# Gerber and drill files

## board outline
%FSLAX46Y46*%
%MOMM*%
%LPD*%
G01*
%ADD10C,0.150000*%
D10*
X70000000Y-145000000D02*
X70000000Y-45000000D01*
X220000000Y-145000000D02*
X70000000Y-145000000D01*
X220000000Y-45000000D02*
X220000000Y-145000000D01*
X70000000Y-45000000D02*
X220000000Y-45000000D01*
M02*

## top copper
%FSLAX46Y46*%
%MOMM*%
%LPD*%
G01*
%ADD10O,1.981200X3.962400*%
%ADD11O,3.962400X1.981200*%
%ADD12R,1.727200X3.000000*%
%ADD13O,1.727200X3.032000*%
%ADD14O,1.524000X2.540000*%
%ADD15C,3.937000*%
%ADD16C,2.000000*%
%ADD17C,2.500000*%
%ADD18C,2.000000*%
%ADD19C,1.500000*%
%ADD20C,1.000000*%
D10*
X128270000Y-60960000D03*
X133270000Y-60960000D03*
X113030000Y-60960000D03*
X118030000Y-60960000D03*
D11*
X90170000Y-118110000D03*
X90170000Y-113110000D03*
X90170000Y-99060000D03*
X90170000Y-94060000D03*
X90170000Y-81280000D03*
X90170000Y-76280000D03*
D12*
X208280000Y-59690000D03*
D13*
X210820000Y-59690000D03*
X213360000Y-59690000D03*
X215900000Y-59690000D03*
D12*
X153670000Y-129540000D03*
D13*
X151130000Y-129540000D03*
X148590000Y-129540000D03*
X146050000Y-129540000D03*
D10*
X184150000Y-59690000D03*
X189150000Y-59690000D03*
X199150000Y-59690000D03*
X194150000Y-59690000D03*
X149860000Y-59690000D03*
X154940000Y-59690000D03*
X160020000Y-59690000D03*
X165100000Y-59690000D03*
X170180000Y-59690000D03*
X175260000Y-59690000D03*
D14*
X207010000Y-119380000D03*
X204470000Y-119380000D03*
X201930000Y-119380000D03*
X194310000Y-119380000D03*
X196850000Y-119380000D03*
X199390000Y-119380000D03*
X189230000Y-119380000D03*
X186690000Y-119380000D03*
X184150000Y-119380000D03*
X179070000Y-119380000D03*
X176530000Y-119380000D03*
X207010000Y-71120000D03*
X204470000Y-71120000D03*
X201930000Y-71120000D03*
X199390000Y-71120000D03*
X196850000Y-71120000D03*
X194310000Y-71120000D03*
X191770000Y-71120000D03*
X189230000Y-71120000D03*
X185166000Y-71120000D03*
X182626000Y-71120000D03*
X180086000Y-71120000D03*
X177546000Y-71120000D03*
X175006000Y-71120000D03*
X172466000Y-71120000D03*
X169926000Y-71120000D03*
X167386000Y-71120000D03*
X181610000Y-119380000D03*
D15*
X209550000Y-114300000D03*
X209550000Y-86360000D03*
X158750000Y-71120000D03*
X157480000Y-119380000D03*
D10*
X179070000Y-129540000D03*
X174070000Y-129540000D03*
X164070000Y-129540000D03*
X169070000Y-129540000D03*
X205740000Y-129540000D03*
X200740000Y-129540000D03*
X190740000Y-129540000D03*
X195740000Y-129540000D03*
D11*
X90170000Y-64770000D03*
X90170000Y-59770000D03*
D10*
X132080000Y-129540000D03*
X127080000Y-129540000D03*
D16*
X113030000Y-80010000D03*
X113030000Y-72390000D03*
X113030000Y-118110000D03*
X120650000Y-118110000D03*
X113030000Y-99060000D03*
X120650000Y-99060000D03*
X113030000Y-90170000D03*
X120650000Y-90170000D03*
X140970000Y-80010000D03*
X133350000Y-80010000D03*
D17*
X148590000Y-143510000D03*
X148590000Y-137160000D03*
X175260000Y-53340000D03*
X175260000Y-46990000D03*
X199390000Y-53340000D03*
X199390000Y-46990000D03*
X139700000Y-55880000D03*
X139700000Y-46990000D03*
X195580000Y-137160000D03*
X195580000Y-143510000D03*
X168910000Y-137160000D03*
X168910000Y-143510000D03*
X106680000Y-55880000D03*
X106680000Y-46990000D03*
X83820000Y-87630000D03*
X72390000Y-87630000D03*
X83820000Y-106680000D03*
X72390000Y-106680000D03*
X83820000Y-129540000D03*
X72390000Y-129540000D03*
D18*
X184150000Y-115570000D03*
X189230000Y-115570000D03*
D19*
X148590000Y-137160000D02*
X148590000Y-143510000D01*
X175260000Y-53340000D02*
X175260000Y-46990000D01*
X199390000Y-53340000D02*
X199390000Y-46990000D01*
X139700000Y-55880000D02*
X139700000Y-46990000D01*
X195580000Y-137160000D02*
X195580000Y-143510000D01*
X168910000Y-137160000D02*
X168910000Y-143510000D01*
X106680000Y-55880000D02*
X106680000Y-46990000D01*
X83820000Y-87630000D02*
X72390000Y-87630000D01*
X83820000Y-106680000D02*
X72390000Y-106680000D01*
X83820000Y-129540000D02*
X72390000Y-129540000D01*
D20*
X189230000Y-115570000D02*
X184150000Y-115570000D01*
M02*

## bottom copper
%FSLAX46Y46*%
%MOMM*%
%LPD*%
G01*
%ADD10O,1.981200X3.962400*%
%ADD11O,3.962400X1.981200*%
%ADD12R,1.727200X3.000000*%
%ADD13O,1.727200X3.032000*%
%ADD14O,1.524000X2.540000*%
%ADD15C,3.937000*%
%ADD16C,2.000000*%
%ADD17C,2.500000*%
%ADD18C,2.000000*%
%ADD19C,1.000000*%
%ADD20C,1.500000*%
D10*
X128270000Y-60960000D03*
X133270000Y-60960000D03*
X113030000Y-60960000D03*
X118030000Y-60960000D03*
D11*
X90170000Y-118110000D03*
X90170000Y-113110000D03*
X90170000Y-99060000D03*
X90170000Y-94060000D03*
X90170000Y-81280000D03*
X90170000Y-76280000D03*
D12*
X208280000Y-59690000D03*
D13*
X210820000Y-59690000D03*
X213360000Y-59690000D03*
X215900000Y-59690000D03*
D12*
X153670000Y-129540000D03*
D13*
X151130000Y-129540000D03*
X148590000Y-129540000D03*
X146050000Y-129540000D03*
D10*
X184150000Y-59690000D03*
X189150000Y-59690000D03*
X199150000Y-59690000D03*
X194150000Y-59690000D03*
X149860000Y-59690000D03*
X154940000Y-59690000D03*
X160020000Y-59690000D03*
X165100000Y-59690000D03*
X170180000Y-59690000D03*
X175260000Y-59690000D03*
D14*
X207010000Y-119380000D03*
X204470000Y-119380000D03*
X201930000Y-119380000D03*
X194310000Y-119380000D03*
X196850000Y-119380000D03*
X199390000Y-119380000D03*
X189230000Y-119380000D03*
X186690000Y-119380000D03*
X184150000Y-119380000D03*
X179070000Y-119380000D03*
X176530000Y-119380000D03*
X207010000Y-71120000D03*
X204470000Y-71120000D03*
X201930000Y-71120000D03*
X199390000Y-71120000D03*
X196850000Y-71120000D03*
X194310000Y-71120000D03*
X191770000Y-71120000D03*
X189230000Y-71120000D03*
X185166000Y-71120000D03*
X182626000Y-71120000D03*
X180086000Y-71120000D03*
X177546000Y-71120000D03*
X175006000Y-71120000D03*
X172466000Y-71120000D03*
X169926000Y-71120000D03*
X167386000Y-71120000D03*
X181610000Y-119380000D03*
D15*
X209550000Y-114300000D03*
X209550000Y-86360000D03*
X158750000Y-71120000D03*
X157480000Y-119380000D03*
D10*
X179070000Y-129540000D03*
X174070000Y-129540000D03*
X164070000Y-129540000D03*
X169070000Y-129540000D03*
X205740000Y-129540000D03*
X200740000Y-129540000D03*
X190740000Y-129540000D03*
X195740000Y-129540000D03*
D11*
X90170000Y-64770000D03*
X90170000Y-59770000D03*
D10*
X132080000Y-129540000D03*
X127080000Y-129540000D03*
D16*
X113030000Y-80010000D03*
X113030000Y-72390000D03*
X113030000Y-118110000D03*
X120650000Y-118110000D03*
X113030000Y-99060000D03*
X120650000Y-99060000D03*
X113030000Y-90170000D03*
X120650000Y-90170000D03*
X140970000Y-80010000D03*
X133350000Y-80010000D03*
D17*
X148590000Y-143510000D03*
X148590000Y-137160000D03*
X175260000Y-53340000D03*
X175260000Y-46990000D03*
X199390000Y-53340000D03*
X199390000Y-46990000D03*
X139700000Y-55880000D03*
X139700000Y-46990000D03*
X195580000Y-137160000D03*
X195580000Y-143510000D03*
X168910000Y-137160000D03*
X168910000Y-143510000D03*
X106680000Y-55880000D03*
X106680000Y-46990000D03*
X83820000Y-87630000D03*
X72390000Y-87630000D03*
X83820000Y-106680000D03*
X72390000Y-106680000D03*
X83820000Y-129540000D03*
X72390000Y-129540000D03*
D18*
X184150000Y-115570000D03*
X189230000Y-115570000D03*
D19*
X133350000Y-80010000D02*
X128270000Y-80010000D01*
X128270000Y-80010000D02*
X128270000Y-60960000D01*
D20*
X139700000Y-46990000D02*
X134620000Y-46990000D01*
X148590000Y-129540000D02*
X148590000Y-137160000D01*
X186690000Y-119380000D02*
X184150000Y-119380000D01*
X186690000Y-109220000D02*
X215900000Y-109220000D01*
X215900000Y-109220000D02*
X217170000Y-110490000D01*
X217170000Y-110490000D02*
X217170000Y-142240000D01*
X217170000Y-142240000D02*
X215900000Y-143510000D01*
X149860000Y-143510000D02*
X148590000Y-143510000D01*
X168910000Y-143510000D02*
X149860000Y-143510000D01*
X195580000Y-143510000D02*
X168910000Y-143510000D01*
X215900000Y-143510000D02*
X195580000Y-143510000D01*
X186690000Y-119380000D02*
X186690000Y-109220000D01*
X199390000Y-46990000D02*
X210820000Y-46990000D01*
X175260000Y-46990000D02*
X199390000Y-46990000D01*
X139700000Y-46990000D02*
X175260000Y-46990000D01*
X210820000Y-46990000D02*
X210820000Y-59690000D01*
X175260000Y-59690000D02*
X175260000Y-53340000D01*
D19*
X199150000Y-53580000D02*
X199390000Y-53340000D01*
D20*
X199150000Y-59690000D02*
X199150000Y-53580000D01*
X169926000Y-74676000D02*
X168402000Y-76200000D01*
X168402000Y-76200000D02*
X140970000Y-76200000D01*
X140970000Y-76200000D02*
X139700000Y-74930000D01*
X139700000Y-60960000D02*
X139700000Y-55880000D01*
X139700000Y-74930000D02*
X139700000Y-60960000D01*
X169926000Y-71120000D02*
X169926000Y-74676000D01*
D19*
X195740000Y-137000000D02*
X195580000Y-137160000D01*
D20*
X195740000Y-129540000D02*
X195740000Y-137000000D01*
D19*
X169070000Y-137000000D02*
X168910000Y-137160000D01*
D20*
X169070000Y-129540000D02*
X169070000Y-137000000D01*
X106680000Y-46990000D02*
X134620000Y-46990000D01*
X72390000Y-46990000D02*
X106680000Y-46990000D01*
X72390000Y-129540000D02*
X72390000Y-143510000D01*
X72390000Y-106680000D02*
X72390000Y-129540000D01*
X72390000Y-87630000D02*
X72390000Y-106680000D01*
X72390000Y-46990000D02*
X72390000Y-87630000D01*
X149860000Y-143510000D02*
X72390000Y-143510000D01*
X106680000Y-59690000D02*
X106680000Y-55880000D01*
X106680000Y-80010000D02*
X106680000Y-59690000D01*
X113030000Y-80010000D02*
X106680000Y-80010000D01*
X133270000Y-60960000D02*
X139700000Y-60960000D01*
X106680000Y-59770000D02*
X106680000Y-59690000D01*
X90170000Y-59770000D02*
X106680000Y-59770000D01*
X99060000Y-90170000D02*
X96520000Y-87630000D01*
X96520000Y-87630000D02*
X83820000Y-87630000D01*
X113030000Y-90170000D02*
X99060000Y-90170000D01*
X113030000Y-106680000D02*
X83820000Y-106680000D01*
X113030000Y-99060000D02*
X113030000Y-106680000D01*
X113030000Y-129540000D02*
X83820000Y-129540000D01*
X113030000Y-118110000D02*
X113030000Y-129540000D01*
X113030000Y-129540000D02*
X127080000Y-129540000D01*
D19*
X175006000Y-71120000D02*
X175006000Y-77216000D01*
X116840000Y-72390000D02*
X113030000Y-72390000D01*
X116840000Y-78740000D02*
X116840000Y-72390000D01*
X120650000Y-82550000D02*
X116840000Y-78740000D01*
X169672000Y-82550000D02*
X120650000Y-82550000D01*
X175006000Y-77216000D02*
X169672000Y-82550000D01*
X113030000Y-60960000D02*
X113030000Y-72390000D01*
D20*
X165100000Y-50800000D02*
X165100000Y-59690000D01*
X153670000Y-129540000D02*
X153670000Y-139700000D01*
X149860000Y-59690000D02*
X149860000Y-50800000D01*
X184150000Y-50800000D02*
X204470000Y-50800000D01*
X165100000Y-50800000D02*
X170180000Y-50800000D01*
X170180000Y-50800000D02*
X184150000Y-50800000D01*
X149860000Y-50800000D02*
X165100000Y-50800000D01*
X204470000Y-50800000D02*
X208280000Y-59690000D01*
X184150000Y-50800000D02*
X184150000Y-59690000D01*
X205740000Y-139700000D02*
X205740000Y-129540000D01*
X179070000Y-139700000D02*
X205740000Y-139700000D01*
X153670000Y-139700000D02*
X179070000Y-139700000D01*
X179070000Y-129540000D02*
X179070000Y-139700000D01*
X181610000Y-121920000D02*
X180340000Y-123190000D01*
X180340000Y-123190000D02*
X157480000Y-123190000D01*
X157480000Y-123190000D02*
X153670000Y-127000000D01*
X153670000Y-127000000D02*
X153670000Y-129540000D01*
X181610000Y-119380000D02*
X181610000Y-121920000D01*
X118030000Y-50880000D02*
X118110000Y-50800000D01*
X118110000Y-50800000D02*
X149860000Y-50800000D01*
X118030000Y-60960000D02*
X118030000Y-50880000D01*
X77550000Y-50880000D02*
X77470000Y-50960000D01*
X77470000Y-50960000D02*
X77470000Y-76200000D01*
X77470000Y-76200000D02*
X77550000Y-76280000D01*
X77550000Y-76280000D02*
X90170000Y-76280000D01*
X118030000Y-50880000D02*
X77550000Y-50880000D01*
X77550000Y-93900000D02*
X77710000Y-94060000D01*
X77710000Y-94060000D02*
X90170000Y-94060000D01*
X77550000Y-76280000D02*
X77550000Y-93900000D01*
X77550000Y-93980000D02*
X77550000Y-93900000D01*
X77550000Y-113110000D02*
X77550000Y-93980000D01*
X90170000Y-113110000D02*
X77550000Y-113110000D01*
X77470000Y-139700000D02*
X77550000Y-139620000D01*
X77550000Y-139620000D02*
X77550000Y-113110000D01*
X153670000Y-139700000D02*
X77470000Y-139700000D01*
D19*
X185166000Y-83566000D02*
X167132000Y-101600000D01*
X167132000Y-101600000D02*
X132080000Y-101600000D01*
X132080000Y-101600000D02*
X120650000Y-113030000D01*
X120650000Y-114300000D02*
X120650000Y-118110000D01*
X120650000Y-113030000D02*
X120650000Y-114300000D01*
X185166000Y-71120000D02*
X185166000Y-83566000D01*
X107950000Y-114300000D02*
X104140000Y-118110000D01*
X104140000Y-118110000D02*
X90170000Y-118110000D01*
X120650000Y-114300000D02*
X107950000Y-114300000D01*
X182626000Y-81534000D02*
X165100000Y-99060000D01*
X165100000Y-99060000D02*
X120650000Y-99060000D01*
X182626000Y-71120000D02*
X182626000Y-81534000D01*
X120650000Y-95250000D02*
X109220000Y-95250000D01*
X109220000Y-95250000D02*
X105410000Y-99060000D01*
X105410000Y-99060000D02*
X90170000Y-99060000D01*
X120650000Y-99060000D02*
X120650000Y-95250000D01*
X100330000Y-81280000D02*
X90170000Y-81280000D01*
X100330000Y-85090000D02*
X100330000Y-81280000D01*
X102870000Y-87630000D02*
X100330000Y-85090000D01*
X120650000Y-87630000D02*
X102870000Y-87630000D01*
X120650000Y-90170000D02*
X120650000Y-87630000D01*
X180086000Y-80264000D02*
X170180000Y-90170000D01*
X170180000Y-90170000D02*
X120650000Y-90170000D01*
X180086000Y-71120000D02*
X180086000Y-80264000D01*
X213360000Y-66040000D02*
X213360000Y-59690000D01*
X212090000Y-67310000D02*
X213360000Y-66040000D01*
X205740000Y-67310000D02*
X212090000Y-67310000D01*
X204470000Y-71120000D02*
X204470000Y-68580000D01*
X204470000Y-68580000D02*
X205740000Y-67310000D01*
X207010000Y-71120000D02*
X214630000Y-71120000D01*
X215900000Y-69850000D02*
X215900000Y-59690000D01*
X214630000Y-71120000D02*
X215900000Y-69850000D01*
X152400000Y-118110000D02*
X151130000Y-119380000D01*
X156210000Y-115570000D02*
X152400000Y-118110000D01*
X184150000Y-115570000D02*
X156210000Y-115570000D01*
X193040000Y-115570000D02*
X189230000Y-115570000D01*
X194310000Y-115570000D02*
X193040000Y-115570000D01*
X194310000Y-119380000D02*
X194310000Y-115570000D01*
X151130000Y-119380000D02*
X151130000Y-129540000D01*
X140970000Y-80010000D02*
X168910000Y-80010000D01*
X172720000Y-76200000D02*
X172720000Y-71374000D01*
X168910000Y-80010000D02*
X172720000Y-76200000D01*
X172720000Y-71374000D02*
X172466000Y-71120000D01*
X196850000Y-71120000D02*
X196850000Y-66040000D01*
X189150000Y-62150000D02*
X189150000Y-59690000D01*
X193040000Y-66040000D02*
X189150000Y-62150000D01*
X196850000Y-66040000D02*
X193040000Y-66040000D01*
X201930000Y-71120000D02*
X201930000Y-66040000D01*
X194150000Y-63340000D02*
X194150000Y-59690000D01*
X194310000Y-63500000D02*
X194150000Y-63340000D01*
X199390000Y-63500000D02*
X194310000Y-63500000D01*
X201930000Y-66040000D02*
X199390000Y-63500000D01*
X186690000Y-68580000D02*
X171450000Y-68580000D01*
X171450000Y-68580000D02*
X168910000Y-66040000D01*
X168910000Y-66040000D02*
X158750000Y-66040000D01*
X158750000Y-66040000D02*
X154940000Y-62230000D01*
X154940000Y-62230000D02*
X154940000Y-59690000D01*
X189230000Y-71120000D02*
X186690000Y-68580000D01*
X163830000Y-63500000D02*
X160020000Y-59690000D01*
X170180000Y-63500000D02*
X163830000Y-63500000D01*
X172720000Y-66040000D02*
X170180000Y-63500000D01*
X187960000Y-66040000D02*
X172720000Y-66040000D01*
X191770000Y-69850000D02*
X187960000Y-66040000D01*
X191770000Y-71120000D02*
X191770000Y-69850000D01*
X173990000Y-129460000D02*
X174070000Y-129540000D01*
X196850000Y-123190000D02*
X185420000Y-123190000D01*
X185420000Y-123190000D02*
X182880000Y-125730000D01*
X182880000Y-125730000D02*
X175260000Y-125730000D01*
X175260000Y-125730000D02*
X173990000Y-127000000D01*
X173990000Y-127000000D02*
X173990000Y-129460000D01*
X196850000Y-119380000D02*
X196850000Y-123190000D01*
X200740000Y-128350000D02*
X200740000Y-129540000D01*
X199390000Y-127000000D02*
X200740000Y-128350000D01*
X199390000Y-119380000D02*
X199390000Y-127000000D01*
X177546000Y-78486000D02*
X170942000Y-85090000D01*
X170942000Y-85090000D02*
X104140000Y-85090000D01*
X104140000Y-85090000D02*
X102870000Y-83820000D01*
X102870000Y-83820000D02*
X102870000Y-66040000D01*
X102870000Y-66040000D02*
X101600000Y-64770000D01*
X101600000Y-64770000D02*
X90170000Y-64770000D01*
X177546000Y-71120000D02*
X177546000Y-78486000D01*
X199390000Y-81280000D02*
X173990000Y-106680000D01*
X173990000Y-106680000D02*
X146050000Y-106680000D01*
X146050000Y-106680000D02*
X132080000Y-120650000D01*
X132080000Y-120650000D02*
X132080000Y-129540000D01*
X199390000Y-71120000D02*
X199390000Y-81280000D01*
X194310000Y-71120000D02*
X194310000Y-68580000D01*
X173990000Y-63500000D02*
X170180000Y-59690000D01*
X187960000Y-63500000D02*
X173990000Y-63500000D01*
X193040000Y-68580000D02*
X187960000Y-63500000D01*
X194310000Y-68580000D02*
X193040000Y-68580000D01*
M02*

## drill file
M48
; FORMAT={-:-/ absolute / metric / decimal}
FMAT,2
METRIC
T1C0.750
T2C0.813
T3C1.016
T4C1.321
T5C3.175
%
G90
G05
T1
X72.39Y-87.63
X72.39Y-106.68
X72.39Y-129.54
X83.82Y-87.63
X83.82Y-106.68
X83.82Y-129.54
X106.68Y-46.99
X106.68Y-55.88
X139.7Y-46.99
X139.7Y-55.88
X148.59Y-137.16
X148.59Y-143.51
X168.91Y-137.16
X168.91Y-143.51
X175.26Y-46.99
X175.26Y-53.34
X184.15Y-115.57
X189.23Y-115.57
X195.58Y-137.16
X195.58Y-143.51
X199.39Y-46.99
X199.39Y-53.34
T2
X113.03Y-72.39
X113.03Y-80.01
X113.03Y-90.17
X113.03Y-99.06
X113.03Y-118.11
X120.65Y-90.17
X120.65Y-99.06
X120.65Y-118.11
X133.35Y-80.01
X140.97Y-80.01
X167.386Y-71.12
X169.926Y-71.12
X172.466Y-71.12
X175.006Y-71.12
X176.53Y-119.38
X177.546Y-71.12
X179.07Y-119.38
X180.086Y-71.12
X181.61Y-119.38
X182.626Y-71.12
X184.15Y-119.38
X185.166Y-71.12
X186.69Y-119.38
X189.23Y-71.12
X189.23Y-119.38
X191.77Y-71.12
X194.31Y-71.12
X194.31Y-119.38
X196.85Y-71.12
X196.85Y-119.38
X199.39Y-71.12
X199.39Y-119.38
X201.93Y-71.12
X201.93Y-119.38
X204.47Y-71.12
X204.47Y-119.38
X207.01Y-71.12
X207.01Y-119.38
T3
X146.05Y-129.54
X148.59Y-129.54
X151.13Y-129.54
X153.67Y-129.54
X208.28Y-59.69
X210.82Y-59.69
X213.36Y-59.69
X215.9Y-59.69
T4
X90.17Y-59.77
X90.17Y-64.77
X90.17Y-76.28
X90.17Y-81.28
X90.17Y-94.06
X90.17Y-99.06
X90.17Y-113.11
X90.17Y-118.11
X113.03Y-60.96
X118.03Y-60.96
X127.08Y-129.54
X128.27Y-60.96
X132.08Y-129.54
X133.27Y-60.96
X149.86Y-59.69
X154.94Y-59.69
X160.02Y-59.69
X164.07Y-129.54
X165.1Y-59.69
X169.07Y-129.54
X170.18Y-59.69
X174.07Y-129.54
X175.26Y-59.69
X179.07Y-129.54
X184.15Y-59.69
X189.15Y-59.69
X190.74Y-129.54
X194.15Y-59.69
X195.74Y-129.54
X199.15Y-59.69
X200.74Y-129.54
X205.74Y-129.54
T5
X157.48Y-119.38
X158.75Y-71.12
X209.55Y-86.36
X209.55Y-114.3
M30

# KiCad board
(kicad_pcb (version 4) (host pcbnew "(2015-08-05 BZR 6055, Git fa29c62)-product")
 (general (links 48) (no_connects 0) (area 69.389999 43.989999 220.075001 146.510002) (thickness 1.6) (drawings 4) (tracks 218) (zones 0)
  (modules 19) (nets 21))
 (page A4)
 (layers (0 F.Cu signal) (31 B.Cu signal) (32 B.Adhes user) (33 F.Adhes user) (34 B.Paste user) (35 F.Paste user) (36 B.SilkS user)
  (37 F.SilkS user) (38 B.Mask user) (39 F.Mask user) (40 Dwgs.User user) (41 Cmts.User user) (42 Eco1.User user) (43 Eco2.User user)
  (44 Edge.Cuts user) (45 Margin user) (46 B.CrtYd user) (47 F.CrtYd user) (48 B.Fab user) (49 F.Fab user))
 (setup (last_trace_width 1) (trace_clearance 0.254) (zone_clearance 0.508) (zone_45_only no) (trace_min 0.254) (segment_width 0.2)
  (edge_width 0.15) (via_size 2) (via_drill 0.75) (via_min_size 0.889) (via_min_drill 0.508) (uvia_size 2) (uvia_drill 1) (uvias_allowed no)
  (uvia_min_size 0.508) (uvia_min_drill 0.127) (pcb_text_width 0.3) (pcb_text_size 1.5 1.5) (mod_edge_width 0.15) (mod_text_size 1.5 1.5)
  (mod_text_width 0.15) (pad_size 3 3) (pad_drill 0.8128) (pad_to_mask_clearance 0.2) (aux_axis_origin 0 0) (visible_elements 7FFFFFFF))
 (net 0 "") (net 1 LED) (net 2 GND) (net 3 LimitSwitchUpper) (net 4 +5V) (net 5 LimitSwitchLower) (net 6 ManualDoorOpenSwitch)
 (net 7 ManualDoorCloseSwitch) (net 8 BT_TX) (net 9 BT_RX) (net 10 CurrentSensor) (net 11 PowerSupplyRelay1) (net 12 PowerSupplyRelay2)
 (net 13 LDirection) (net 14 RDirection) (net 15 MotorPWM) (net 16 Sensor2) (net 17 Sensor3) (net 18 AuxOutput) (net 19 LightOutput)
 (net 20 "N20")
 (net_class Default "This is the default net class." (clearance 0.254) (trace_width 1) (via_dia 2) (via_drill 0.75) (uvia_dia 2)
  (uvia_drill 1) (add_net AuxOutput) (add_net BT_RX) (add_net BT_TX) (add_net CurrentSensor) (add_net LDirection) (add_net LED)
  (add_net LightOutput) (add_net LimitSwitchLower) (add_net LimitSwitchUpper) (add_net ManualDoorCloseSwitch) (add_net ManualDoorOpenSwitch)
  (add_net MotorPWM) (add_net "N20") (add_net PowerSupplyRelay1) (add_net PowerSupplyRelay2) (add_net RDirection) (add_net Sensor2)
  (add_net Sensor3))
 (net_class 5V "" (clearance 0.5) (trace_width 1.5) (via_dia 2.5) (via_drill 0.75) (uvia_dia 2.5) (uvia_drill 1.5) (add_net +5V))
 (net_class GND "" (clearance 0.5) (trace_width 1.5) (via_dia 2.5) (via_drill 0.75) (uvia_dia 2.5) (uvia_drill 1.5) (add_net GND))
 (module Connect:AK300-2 (layer F.Cu) (at 128.27 60.96)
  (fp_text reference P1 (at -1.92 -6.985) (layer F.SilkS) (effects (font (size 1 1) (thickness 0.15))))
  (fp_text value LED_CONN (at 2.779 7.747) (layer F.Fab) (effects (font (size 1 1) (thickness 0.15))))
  (pad 1 thru_hole oval (at 0 0) (size 1.9812 3.9624) (drill 1.3208) (layers *.Cu F.Paste F.SilkS F.Mask) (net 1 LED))
  (pad 2 thru_hole oval (at 5 0) (size 1.9812 3.9624) (drill 1.3208) (layers *.Cu F.Paste F.SilkS F.Mask) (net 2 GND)))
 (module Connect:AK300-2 (layer F.Cu) (at 113.03 60.96)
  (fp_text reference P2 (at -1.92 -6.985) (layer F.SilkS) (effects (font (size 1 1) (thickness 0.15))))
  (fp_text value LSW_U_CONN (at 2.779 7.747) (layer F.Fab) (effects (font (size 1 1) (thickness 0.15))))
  (pad 1 thru_hole oval (at 0 0) (size 1.9812 3.9624) (drill 1.3208) (layers *.Cu F.Paste F.SilkS F.Mask) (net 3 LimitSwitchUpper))
  (pad 2 thru_hole oval (at 5 0) (size 1.9812 3.9624) (drill 1.3208) (layers *.Cu F.Paste F.SilkS F.Mask) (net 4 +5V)))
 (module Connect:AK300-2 (layer F.Cu) (at 90.17 118.11 90)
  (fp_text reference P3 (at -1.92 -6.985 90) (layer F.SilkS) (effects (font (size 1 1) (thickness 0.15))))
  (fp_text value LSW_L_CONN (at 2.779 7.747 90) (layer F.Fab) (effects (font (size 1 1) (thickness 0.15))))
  (pad 1 thru_hole oval (at 0 0 90) (size 1.9812 3.9624) (drill 1.3208) (layers *.Cu F.Paste F.SilkS F.Mask) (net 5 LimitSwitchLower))
  (pad 2 thru_hole oval (at 5 0 90) (size 1.9812 3.9624) (drill 1.3208) (layers *.Cu F.Paste F.SilkS F.Mask) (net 4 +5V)))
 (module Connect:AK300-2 (layer F.Cu) (at 90.17 99.06 90)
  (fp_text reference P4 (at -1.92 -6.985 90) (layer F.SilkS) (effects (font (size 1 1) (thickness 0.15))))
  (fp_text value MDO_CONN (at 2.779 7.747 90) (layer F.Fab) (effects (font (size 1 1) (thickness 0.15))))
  (pad 1 thru_hole oval (at 0 0 90) (size 1.9812 3.9624) (drill 1.3208) (layers *.Cu F.Paste F.SilkS F.Mask) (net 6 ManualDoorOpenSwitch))
  (pad 2 thru_hole oval (at 5 0 90) (size 1.9812 3.9624) (drill 1.3208) (layers *.Cu F.Paste F.SilkS F.Mask) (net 4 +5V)))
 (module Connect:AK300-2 (layer F.Cu) (at 90.17 81.28 90)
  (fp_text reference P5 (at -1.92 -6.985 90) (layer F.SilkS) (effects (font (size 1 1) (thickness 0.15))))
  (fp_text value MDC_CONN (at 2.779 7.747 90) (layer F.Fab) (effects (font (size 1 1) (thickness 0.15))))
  (pad 1 thru_hole oval (at 0 0 90) (size 1.9812 3.9624) (drill 1.3208) (layers *.Cu F.Paste F.SilkS F.Mask) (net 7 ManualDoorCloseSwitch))
  (pad 2 thru_hole oval (at 5 0 90) (size 1.9812 3.9624) (drill 1.3208) (layers *.Cu F.Paste F.SilkS F.Mask) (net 4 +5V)))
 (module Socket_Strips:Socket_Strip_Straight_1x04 (layer F.Cu) (at 208.28 59.69)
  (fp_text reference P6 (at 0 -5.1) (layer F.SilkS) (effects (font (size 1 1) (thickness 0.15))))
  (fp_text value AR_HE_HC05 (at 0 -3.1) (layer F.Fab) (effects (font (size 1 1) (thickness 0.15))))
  (pad 1 thru_hole rect (at 0 0) (size 1.7272 3) (drill 1.016) (layers *.Cu *.Mask F.SilkS) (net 4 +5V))
  (pad 2 thru_hole oval (at 2.54 0) (size 1.7272 3.032) (drill 1.016) (layers *.Cu *.Mask F.SilkS) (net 2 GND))
  (pad 3 thru_hole oval (at 5.08 0) (size 1.7272 3.032) (drill 1.016) (layers *.Cu *.Mask F.SilkS) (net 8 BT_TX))
  (pad 4 thru_hole oval (at 7.62 0) (size 1.7272 3.032) (drill 1.016) (layers *.Cu *.Mask F.SilkS) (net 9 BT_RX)))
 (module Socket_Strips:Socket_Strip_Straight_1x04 (layer F.Cu) (at 153.67 129.54 180)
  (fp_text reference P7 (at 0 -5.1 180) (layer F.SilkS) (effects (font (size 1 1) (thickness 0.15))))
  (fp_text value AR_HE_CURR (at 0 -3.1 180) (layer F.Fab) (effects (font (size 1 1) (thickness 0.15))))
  (pad 1 thru_hole rect (at 0 0 180) (size 1.7272 3) (drill 1.016) (layers *.Cu *.Mask F.SilkS) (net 4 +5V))
  (pad 2 thru_hole oval (at 2.54 0 180) (size 1.7272 3.032) (drill 1.016) (layers *.Cu *.Mask F.SilkS) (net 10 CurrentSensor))
  (pad 3 thru_hole oval (at 5.08 0 180) (size 1.7272 3.032) (drill 1.016) (layers *.Cu *.Mask F.SilkS) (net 2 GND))
  (pad 4 thru_hole oval (at 7.62 0 180) (size 1.7272 3.032) (drill 1.016) (layers *.Cu *.Mask F.SilkS)))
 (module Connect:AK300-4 (layer F.Cu) (at 184.15 59.69)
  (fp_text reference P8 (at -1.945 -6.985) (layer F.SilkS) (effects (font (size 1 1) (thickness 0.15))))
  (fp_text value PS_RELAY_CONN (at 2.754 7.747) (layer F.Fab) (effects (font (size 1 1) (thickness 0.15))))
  (pad 1 thru_hole oval (at 0 0) (size 1.9812 3.9624) (drill 1.3208) (layers *.Cu F.Paste F.SilkS F.Mask) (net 4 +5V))
  (pad 2 thru_hole oval (at 5 0) (size 1.9812 3.9624) (drill 1.3208) (layers *.Cu F.Paste F.SilkS F.Mask) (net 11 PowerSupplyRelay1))
  (pad 4 thru_hole oval (at 15 0) (size 1.9812 3.9624) (drill 1.3208) (layers *.Cu F.Paste F.SilkS F.Mask) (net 2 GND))
  (pad 3 thru_hole oval (at 10 0) (size 1.9812 3.9624) (drill 1.3208) (layers *.Cu *.Mask F.SilkS) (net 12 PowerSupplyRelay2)))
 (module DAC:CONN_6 (layer F.Cu) (at 162.56 59.69)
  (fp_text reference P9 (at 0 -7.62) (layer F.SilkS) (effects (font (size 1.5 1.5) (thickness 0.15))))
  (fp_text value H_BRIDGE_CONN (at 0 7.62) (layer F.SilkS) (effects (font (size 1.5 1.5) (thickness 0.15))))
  (pad 1 thru_hole oval (at -12.7 0) (size 1.9812 3.9624) (drill 1.3208) (layers *.Cu *.Mask F.SilkS) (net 4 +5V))
  (pad 2 thru_hole oval (at -7.62 0) (size 1.9812 3.9624) (drill 1.3208) (layers *.Cu *.Mask F.SilkS) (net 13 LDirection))
  (pad 3 thru_hole oval (at -2.54 0) (size 1.9812 3.9624) (drill 1.3208) (layers *.Cu *.Mask F.SilkS) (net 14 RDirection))
  (pad 4 thru_hole oval (at 2.54 0) (size 1.9812 3.9624) (drill 1.3208) (layers *.Cu *.Mask F.SilkS) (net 4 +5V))
  (pad 5 thru_hole oval (at 7.62 0) (size 1.9812 3.9624) (drill 1.3208) (layers *.Cu *.Mask F.SilkS) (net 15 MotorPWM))
  (pad 6 thru_hole oval (at 12.7 0) (size 1.9812 3.9624) (drill 1.3208) (layers *.Cu *.Mask F.SilkS) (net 2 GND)))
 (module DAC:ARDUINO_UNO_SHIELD (layer F.Cu) (at 143.51 121.92)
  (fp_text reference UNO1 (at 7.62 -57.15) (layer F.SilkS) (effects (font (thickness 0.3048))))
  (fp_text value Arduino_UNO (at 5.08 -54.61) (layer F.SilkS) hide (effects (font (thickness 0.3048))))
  (pad AD5 thru_hole oval (at 63.5 -2.54 90) (size 2.54 1.524) (drill 0.8128) (layers *.Cu *.Mask F.SilkS))
  (pad AD4 thru_hole oval (at 60.96 -2.54 90) (size 2.54 1.524) (drill 0.8128) (layers *.Cu *.Mask F.SilkS))
  (pad AD3 thru_hole oval (at 58.42 -2.54 90) (size 2.54 1.524) (drill 0.8128) (layers *.Cu *.Mask F.SilkS))
  (pad AD0 thru_hole oval (at 50.8 -2.54 90) (size 2.54 1.524) (drill 0.8128) (layers *.Cu *.Mask F.SilkS) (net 10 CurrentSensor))
  (pad AD1 thru_hole oval (at 53.34 -2.54 90) (size 2.54 1.524) (drill 0.8128) (layers *.Cu *.Mask F.SilkS) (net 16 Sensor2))
  (pad AD2 thru_hole oval (at 55.88 -2.54 90) (size 2.54 1.524) (drill 0.8128) (layers *.Cu *.Mask F.SilkS) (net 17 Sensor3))
  (pad V_IN thru_hole oval (at 45.72 -2.54 90) (size 2.54 1.524) (drill 0.8128) (layers *.Cu *.Mask F.SilkS))
  (pad GND2 thru_hole oval (at 43.18 -2.54 90) (size 2.54 1.524) (drill 0.8128) (layers *.Cu *.Mask F.SilkS) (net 2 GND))
  (pad GND1 thru_hole oval (at 40.64 -2.54 90) (size 2.54 1.524) (drill 0.8128) (layers *.Cu *.Mask F.SilkS) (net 2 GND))
  (pad 3V3 thru_hole oval (at 35.56 -2.54 90) (size 2.54 1.524) (drill 0.8128) (layers *.Cu *.Mask F.SilkS))
  (pad RST thru_hole oval (at 33.02 -2.54 90) (size 2.54 1.524) (drill 0.8128) (layers *.Cu *.Mask F.SilkS))
  (pad 0 thru_hole oval (at 63.5 -50.8 90) (size 2.54 1.524) (drill 0.8128) (layers *.Cu *.Mask F.SilkS) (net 9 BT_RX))
  (pad 1 thru_hole oval (at 60.96 -50.8 90) (size 2.54 1.524) (drill 0.8128) (layers *.Cu *.Mask F.SilkS) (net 8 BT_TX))
  (pad 2 thru_hole oval (at 58.42 -50.8 90) (size 2.54 1.524) (drill 0.8128) (layers *.Cu *.Mask F.SilkS) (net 12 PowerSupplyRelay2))
  (pad 3 thru_hole oval (at 55.88 -50.8 90) (size 2.54 1.524) (drill 0.8128) (layers *.Cu *.Mask F.SilkS) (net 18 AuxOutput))
  (pad 4 thru_hole oval (at 53.34 -50.8 90) (size 2.54 1.524) (drill 0.8128) (layers *.Cu *.Mask F.SilkS) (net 11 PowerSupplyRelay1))
  (pad 5 thru_hole oval (at 50.8 -50.8 90) (size 2.54 1.524) (drill 0.8128) (layers *.Cu *.Mask F.SilkS) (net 15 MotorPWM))
  (pad 6 thru_hole oval (at 48.26 -50.8 90) (size 2.54 1.524) (drill 0.8128) (layers *.Cu *.Mask F.SilkS) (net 14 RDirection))
  (pad 7 thru_hole oval (at 45.72 -50.8 90) (size 2.54 1.524) (drill 0.8128) (layers *.Cu *.Mask F.SilkS) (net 13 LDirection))
  (pad 8 thru_hole oval (at 41.656 -50.8 90) (size 2.54 1.524) (drill 0.8128) (layers *.Cu *.Mask F.SilkS) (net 5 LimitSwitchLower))
  (pad 9 thru_hole oval (at 39.116 -50.8 90) (size 2.54 1.524) (drill 0.8128) (layers *.Cu *.Mask F.SilkS) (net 6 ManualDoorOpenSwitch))
  (pad 10 thru_hole oval (at 36.576 -50.8 90) (size 2.54 1.524) (drill 0.8128) (layers *.Cu *.Mask F.SilkS) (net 7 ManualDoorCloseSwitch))
  (pad 11 thru_hole oval (at 34.036 -50.8 90) (size 2.54 1.524) (drill 0.8128) (layers *.Cu *.Mask F.SilkS) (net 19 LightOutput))
  (pad 12 thru_hole oval (at 31.496 -50.8 90) (size 2.54 1.524) (drill 0.8128) (layers *.Cu *.Mask F.SilkS) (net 3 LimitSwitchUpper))
  (pad 13 thru_hole oval (at 28.956 -50.8 90) (size 2.54 1.524) (drill 0.8128) (layers *.Cu *.Mask F.SilkS) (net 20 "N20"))
  (pad GND3 thru_hole oval (at 26.416 -50.8 90) (size 2.54 1.524) (drill 0.8128) (layers *.Cu *.Mask F.SilkS) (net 2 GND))
  (pad AREF thru_hole oval (at 23.876 -50.8 90) (size 2.54 1.524) (drill 0.8128) (layers *.Cu *.Mask F.SilkS))
  (pad 5V thru_hole oval (at 38.1 -2.54 90) (size 2.54 1.524) (drill 0.8128) (layers *.Cu *.Mask F.SilkS) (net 4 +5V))
  (pad "" thru_hole circle (at 66.04 -7.62 90) (size 3.937 3.937) (drill 3.175) (layers *.Cu *.Mask F.SilkS))
  (pad "" thru_hole circle (at 66.04 -35.56 90) (size 3.937 3.937) (drill 3.175) (layers *.Cu *.Mask F.SilkS))
  (pad "" thru_hole circle (at 15.24 -50.8 90) (size 3.937 3.937) (drill 3.175) (layers *.Cu *.Mask F.SilkS))
  (pad "" thru_hole circle (at 13.97 -2.54 90) (size 3.937 3.937) (drill 3.175) (layers *.Cu *.Mask F.SilkS)))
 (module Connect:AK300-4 (layer F.Cu) (at 179.07 129.54 180)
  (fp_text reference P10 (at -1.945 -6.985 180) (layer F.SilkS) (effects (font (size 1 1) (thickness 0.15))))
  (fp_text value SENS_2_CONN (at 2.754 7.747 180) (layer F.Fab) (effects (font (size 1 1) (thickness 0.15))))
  (pad 1 thru_hole oval (at 0 0 180) (size 1.9812 3.9624) (drill 1.3208) (layers *.Cu F.Paste F.SilkS F.Mask) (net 4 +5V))
  (pad 2 thru_hole oval (at 5 0 180) (size 1.9812 3.9624) (drill 1.3208) (layers *.Cu F.Paste F.SilkS F.Mask) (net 16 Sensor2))
  (pad 4 thru_hole oval (at 15 0 180) (size 1.9812 3.9624) (drill 1.3208) (layers *.Cu F.Paste F.SilkS F.Mask))
  (pad 3 thru_hole oval (at 10 0 180) (size 1.9812 3.9624) (drill 1.3208) (layers *.Cu *.Mask F.SilkS) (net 2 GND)))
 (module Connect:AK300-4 (layer F.Cu) (at 205.74 129.54 180)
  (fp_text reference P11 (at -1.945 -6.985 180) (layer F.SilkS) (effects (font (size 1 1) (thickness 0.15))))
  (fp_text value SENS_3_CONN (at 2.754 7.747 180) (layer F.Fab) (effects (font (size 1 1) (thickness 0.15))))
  (pad 1 thru_hole oval (at 0 0 180) (size 1.9812 3.9624) (drill 1.3208) (layers *.Cu F.Paste F.SilkS F.Mask) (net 4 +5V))
  (pad 2 thru_hole oval (at 5 0 180) (size 1.9812 3.9624) (drill 1.3208) (layers *.Cu F.Paste F.SilkS F.Mask) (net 17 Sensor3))
  (pad 4 thru_hole oval (at 15 0 180) (size 1.9812 3.9624) (drill 1.3208) (layers *.Cu F.Paste F.SilkS F.Mask))
  (pad 3 thru_hole oval (at 10 0 180) (size 1.9812 3.9624) (drill 1.3208) (layers *.Cu *.Mask F.SilkS) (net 2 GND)))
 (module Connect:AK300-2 (layer F.Cu) (at 90.17 64.77 90)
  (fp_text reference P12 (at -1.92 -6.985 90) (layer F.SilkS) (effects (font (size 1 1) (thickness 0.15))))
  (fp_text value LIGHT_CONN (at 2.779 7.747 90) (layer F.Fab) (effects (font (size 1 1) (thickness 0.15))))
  (pad 1 thru_hole oval (at 0 0 90) (size 1.9812 3.9624) (drill 1.3208) (layers *.Cu F.Paste F.SilkS F.Mask) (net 19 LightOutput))
  (pad 2 thru_hole oval (at 5 0 90) (size 1.9812 3.9624) (drill 1.3208) (layers *.Cu F.Paste F.SilkS F.Mask) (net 2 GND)))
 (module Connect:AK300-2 (layer F.Cu) (at 132.08 129.54 180)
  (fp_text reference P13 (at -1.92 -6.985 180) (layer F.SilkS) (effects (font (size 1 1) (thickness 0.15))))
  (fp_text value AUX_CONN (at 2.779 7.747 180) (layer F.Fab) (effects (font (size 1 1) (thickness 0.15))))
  (pad 1 thru_hole oval (at 0 0 180) (size 1.9812 3.9624) (drill 1.3208) (layers *.Cu F.Paste F.SilkS F.Mask) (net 18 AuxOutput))
  (pad 2 thru_hole oval (at 5 0 180) (size 1.9812 3.9624) (drill 1.3208) (layers *.Cu F.Paste F.SilkS F.Mask) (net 2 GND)))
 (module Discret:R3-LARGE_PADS (layer F.Cu) (at 113.03 76.2 90)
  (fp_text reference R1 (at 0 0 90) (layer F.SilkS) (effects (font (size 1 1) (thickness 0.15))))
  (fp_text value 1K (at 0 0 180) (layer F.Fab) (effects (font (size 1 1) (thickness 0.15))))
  (pad 1 thru_hole circle (at -3.81 0 90) (size 2 2) (drill 0.8128) (layers *.Cu *.Mask F.SilkS) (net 2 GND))
  (pad 2 thru_hole circle (at 3.81 0 90) (size 2 2) (drill 0.8128) (layers *.Cu *.Mask F.SilkS) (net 3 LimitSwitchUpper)))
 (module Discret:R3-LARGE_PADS (layer F.Cu) (at 116.84 118.11)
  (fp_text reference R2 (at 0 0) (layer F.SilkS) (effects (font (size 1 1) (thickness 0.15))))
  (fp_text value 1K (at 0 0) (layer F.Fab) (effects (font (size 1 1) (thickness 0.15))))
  (pad 1 thru_hole circle (at -3.81 0) (size 2 2) (drill 0.8128) (layers *.Cu *.Mask F.SilkS) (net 2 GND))
  (pad 2 thru_hole circle (at 3.81 0) (size 2 2) (drill 0.8128) (layers *.Cu *.Mask F.SilkS) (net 5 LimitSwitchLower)))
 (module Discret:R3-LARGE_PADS (layer F.Cu) (at 116.84 99.06)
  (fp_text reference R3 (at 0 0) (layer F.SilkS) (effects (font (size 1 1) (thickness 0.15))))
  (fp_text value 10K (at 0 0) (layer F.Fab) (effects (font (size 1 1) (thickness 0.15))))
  (pad 1 thru_hole circle (at -3.81 0) (size 2 2) (drill 0.8128) (layers *.Cu *.Mask F.SilkS) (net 2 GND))
  (pad 2 thru_hole circle (at 3.81 0) (size 2 2) (drill 0.8128) (layers *.Cu *.Mask F.SilkS) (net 6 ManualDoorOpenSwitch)))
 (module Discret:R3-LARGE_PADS (layer F.Cu) (at 116.84 90.17)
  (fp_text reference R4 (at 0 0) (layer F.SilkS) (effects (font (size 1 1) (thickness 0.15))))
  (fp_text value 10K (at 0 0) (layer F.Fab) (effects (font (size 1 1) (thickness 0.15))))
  (pad 1 thru_hole circle (at -3.81 0) (size 2 2) (drill 0.8128) (layers *.Cu *.Mask F.SilkS) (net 2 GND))
  (pad 2 thru_hole circle (at 3.81 0) (size 2 2) (drill 0.8128) (layers *.Cu *.Mask F.SilkS) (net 7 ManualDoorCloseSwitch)))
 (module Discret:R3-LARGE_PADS (layer F.Cu) (at 137.16 80.01 180)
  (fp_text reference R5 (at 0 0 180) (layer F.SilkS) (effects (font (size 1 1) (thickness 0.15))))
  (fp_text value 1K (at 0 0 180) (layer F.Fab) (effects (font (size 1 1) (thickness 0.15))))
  (pad 1 thru_hole circle (at -3.81 0 180) (size 2 2) (drill 0.8128) (layers *.Cu *.Mask F.SilkS) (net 20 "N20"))
  (pad 2 thru_hole circle (at 3.81 0 180) (size 2 2) (drill 0.8128) (layers *.Cu *.Mask F.SilkS) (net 1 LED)))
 (gr_line (start 70 145) (end 70 45) (angle 90) (layer Edge.Cuts) (width 0.15))
 (gr_line (start 220 145) (end 70 145) (angle 90) (layer Edge.Cuts) (width 0.15))
 (gr_line (start 220 45) (end 220 145) (angle 90) (layer Edge.Cuts) (width 0.15))
 (gr_line (start 70 45) (end 220 45) (angle 90) (layer Edge.Cuts) (width 0.15))
 (segment (start 133.35 80.01) (end 128.27 80.01) (width 1) (layer B.Cu) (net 1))
 (segment (start 128.27 80.01) (end 128.27 60.96) (width 1) (layer B.Cu) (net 1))
 (segment (start 139.7 46.99) (end 134.62 46.99) (width 1.5) (layer B.Cu) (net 2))
 (segment (start 148.59 129.54) (end 148.59 137.16) (width 1.5) (layer B.Cu) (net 2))
 (via (at 148.59 143.51) (size 2.5) (layers F.Cu B.Cu) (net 2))
 (segment (start 148.59 137.16) (end 148.59 143.51) (width 1.5) (layer F.Cu) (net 2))
 (via (at 148.59 137.16) (size 2.5) (layers F.Cu B.Cu) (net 2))
 (segment (start 186.69 119.38) (end 184.15 119.38) (width 1.5) (layer B.Cu) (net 2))
 (segment (start 186.69 109.22) (end 215.9 109.22) (width 1.5) (layer B.Cu) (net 2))
 (segment (start 215.9 109.22) (end 217.17 110.49) (width 1.5) (layer B.Cu) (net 2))
 (segment (start 217.17 110.49) (end 217.17 142.24) (width 1.5) (layer B.Cu) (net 2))
 (segment (start 217.17 142.24) (end 215.9 143.51) (width 1.5) (layer B.Cu) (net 2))
 (segment (start 149.86 143.51) (end 148.59 143.51) (width 1.5) (layer B.Cu) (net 2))
 (segment (start 168.91 143.51) (end 149.86 143.51) (width 1.5) (layer B.Cu) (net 2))
 (segment (start 195.58 143.51) (end 168.91 143.51) (width 1.5) (layer B.Cu) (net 2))
 (segment (start 215.9 143.51) (end 195.58 143.51) (width 1.5) (layer B.Cu) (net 2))
 (segment (start 186.69 119.38) (end 186.69 109.22) (width 1.5) (layer B.Cu) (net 2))
 (segment (start 199.39 46.99) (end 210.82 46.99) (width 1.5) (layer B.Cu) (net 2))
 (segment (start 175.26 46.99) (end 199.39 46.99) (width 1.5) (layer B.Cu) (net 2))
 (segment (start 139.7 46.99) (end 175.26 46.99) (width 1.5) (layer B.Cu) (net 2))
 (segment (start 210.82 46.99) (end 210.82 59.69) (width 1.5) (layer B.Cu) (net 2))
 (via (at 175.26 53.34) (size 2.5) (layers F.Cu B.Cu) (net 2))
 (segment (start 175.26 53.34) (end 175.26 46.99) (width 1.5) (layer F.Cu) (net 2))
 (via (at 175.26 46.99) (size 2.5) (layers F.Cu B.Cu) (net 2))
 (segment (start 175.26 59.69) (end 175.26 53.34) (width 1.5) (layer B.Cu) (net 2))
 (segment (start 199.15 53.58) (end 199.39 53.34) (width 1) (layer B.Cu) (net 2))
 (via (at 199.39 53.34) (size 2.5) (layers F.Cu B.Cu) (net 2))
 (segment (start 199.39 53.34) (end 199.39 46.99) (width 1.5) (layer F.Cu) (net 2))
 (via (at 199.39 46.99) (size 2.5) (layers F.Cu B.Cu) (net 2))
 (segment (start 199.15 59.69) (end 199.15 53.58) (width 1.5) (layer B.Cu) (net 2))
 (segment (start 169.926 74.676) (end 168.402 76.2) (width 1.5) (layer B.Cu) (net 2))
 (segment (start 168.402 76.2) (end 140.97 76.2) (width 1.5) (layer B.Cu) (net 2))
 (segment (start 140.97 76.2) (end 139.7 74.93) (width 1.5) (layer B.Cu) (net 2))
 (segment (start 139.7 60.96) (end 139.7 55.88) (width 1.5) (layer B.Cu) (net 2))
 (segment (start 139.7 74.93) (end 139.7 60.96) (width 1.5) (layer B.Cu) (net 2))
 (via (at 139.7 55.88) (size 2.5) (layers F.Cu B.Cu) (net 2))
 (segment (start 139.7 55.88) (end 139.7 46.99) (width 1.5) (layer F.Cu) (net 2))
 (via (at 139.7 46.99) (size 2.5) (layers F.Cu B.Cu) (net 2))
 (segment (start 169.926 71.12) (end 169.926 74.676) (width 1.5) (layer B.Cu) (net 2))
 (segment (start 195.74 137) (end 195.58 137.16) (width 1) (layer B.Cu) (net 2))
 (via (at 195.58 137.16) (size 2.5) (layers F.Cu B.Cu) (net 2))
 (segment (start 195.58 137.16) (end 195.58 143.51) (width 1.5) (layer F.Cu) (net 2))
 (via (at 195.58 143.51) (size 2.5) (layers F.Cu B.Cu) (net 2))
 (segment (start 195.74 129.54) (end 195.74 137) (width 1.5) (layer B.Cu) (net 2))
 (segment (start 169.07 137) (end 168.91 137.16) (width 1) (layer B.Cu) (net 2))
 (via (at 168.91 137.16) (size 2.5) (layers F.Cu B.Cu) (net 2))
 (segment (start 168.91 137.16) (end 168.91 143.51) (width 1.5) (layer F.Cu) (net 2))
 (via (at 168.91 143.51) (size 2.5) (layers F.Cu B.Cu) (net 2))
 (segment (start 169.07 129.54) (end 169.07 137) (width 1.5) (layer B.Cu) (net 2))
 (segment (start 106.68 46.99) (end 134.62 46.99) (width 1.5) (layer B.Cu) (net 2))
 (segment (start 72.39 46.99) (end 106.68 46.99) (width 1.5) (layer B.Cu) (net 2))
 (segment (start 72.39 129.54) (end 72.39 143.51) (width 1.5) (layer B.Cu) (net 2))
 (segment (start 72.39 106.68) (end 72.39 129.54) (width 1.5) (layer B.Cu) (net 2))
 (segment (start 72.39 87.63) (end 72.39 106.68) (width 1.5) (layer B.Cu) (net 2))
 (segment (start 72.39 46.99) (end 72.39 87.63) (width 1.5) (layer B.Cu) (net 2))
 (segment (start 149.86 143.51) (end 72.39 143.51) (width 1.5) (layer B.Cu) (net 2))
 (segment (start 106.68 59.69) (end 106.68 55.88) (width 1.5) (layer B.Cu) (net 2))
 (segment (start 106.68 80.01) (end 106.68 59.69) (width 1.5) (layer B.Cu) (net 2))
 (via (at 106.68 55.88) (size 2.5) (layers F.Cu B.Cu) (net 2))
 (segment (start 106.68 55.88) (end 106.68 46.99) (width 1.5) (layer F.Cu) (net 2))
 (via (at 106.68 46.99) (size 2.5) (layers F.Cu B.Cu) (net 2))
 (segment (start 113.03 80.01) (end 106.68 80.01) (width 1.5) (layer B.Cu) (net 2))
 (segment (start 133.27 60.96) (end 139.7 60.96) (width 1.5) (layer B.Cu) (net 2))
 (segment (start 106.68 59.77) (end 106.68 59.69) (width 1.5) (layer B.Cu) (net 2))
 (segment (start 90.17 59.77) (end 106.68 59.77) (width 1.5) (layer B.Cu) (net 2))
 (segment (start 99.06 90.17) (end 96.52 87.63) (width 1.5) (layer B.Cu) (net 2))
 (segment (start 96.52 87.63) (end 83.82 87.63) (width 1.5) (layer B.Cu) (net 2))
 (via (at 83.82 87.63) (size 2.5) (layers F.Cu B.Cu) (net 2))
 (segment (start 83.82 87.63) (end 72.39 87.63) (width 1.5) (layer F.Cu) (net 2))
 (via (at 72.39 87.63) (size 2.5) (layers F.Cu B.Cu) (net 2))
 (segment (start 113.03 90.17) (end 99.06 90.17) (width 1.5) (layer B.Cu) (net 2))
 (segment (start 113.03 106.68) (end 83.82 106.68) (width 1.5) (layer B.Cu) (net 2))
 (via (at 83.82 106.68) (size 2.5) (layers F.Cu B.Cu) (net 2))
 (segment (start 83.82 106.68) (end 72.39 106.68) (width 1.5) (layer F.Cu) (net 2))
 (via (at 72.39 106.68) (size 2.5) (layers F.Cu B.Cu) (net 2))
 (segment (start 113.03 99.06) (end 113.03 106.68) (width 1.5) (layer B.Cu) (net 2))
 (segment (start 113.03 129.54) (end 83.82 129.54) (width 1.5) (layer B.Cu) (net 2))
 (via (at 83.82 129.54) (size 2.5) (layers F.Cu B.Cu) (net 2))
 (segment (start 83.82 129.54) (end 72.39 129.54) (width 1.5) (layer F.Cu) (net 2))
 (via (at 72.39 129.54) (size 2.5) (layers F.Cu B.Cu) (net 2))
 (segment (start 113.03 118.11) (end 113.03 129.54) (width 1.5) (layer B.Cu) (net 2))
 (segment (start 113.03 129.54) (end 127.08 129.54) (width 1.5) (layer B.Cu) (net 2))
 (segment (start 175.006 71.12) (end 175.006 77.216) (width 1) (layer B.Cu) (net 3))
 (segment (start 116.84 72.39) (end 113.03 72.39) (width 1) (layer B.Cu) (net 3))
 (segment (start 116.84 78.74) (end 116.84 72.39) (width 1) (layer B.Cu) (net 3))
 (segment (start 120.65 82.55) (end 116.84 78.74) (width 1) (layer B.Cu) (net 3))
 (segment (start 169.672 82.55) (end 120.65 82.55) (width 1) (layer B.Cu) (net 3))
 (segment (start 175.006 77.216) (end 169.672 82.55) (width 1) (layer B.Cu) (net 3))
 (segment (start 113.03 60.96) (end 113.03 72.39) (width 1) (layer B.Cu) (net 3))
 (segment (start 165.1 50.8) (end 165.1 59.69) (width 1.5) (layer B.Cu) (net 4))
 (segment (start 153.67 129.54) (end 153.67 139.7) (width 1.5) (layer B.Cu) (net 4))
 (segment (start 149.86 59.69) (end 149.86 50.8) (width 1.5) (layer B.Cu) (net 4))
 (segment (start 184.15 50.8) (end 204.47 50.8) (width 1.5) (layer B.Cu) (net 4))
 (segment (start 165.1 50.8) (end 170.18 50.8) (width 1.5) (layer B.Cu) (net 4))
 (segment (start 170.18 50.8) (end 184.15 50.8) (width 1.5) (layer B.Cu) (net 4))
 (segment (start 149.86 50.8) (end 165.1 50.8) (width 1.5) (layer B.Cu) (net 4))
 (segment (start 204.47 50.8) (end 208.28 59.69) (width 1.5) (layer B.Cu) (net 4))
 (segment (start 184.15 50.8) (end 184.15 59.69) (width 1.5) (layer B.Cu) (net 4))
 (segment (start 205.74 139.7) (end 205.74 129.54) (width 1.5) (layer B.Cu) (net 4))
 (segment (start 179.07 139.7) (end 205.74 139.7) (width 1.5) (layer B.Cu) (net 4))
 (segment (start 153.67 139.7) (end 179.07 139.7) (width 1.5) (layer B.Cu) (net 4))
 (segment (start 179.07 129.54) (end 179.07 139.7) (width 1.5) (layer B.Cu) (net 4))
 (segment (start 181.61 121.92) (end 180.34 123.19) (width 1.5) (layer B.Cu) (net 4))
 (segment (start 180.34 123.19) (end 157.48 123.19) (width 1.5) (layer B.Cu) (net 4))
 (segment (start 157.48 123.19) (end 153.67 127) (width 1.5) (layer B.Cu) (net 4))
 (segment (start 153.67 127) (end 153.67 129.54) (width 1.5) (layer B.Cu) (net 4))
 (segment (start 181.61 119.38) (end 181.61 121.92) (width 1.5) (layer B.Cu) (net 4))
 (segment (start 118.03 50.88) (end 118.11 50.8) (width 1.5) (layer B.Cu) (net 4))
 (segment (start 118.11 50.8) (end 149.86 50.8) (width 1.5) (layer B.Cu) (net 4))
 (segment (start 118.03 60.96) (end 118.03 50.88) (width 1.5) (layer B.Cu) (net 4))
 (segment (start 77.55 50.88) (end 77.47 50.96) (width 1.5) (layer B.Cu) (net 4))
 (segment (start 77.47 50.96) (end 77.47 76.2) (width 1.5) (layer B.Cu) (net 4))
 (segment (start 77.47 76.2) (end 77.55 76.28) (width 1.5) (layer B.Cu) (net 4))
 (segment (start 77.55 76.28) (end 90.17 76.28) (width 1.5) (layer B.Cu) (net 4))
 (segment (start 118.03 50.88) (end 77.55 50.88) (width 1.5) (layer B.Cu) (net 4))
 (segment (start 77.55 93.9) (end 77.71 94.06) (width 1.5) (layer B.Cu) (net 4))
 (segment (start 77.71 94.06) (end 90.17 94.06) (width 1.5) (layer B.Cu) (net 4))
 (segment (start 77.55 76.28) (end 77.55 93.9) (width 1.5) (layer B.Cu) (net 4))
 (segment (start 77.55 93.98) (end 77.55 93.9) (width 1.5) (layer B.Cu) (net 4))
 (segment (start 77.55 113.11) (end 77.55 93.98) (width 1.5) (layer B.Cu) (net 4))
 (segment (start 90.17 113.11) (end 77.55 113.11) (width 1.5) (layer B.Cu) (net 4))
 (segment (start 77.47 139.7) (end 77.55 139.62) (width 1.5) (layer B.Cu) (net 4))
 (segment (start 77.55 139.62) (end 77.55 113.11) (width 1.5) (layer B.Cu) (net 4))
 (segment (start 153.67 139.7) (end 77.47 139.7) (width 1.5) (layer B.Cu) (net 4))
 (segment (start 185.166 83.566) (end 167.132 101.6) (width 1) (layer B.Cu) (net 5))
 (segment (start 167.132 101.6) (end 132.08 101.6) (width 1) (layer B.Cu) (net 5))
 (segment (start 132.08 101.6) (end 120.65 113.03) (width 1) (layer B.Cu) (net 5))
 (segment (start 120.65 114.3) (end 120.65 118.11) (width 1) (layer B.Cu) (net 5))
 (segment (start 120.65 113.03) (end 120.65 114.3) (width 1) (layer B.Cu) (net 5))
 (segment (start 185.166 71.12) (end 185.166 83.566) (width 1) (layer B.Cu) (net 5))
 (segment (start 107.95 114.3) (end 104.14 118.11) (width 1) (layer B.Cu) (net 5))
 (segment (start 104.14 118.11) (end 90.17 118.11) (width 1) (layer B.Cu) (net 5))
 (segment (start 120.65 114.3) (end 107.95 114.3) (width 1) (layer B.Cu) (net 5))
 (segment (start 182.626 81.534) (end 165.1 99.06) (width 1) (layer B.Cu) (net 6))
 (segment (start 165.1 99.06) (end 120.65 99.06) (width 1) (layer B.Cu) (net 6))
 (segment (start 182.626 71.12) (end 182.626 81.534) (width 1) (layer B.Cu) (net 6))
 (segment (start 120.65 95.25) (end 109.22 95.25) (width 1) (layer B.Cu) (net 6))
 (segment (start 109.22 95.25) (end 105.41 99.06) (width 1) (layer B.Cu) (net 6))
 (segment (start 105.41 99.06) (end 90.17 99.06) (width 1) (layer B.Cu) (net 6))
 (segment (start 120.65 99.06) (end 120.65 95.25) (width 1) (layer B.Cu) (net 6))
 (segment (start 100.33 81.28) (end 90.17 81.28) (width 1) (layer B.Cu) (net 7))
 (segment (start 100.33 85.09) (end 100.33 81.28) (width 1) (layer B.Cu) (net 7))
 (segment (start 102.87 87.63) (end 100.33 85.09) (width 1) (layer B.Cu) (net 7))
 (segment (start 120.65 87.63) (end 102.87 87.63) (width 1) (layer B.Cu) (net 7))
 (segment (start 120.65 90.17) (end 120.65 87.63) (width 1) (layer B.Cu) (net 7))
 (segment (start 180.086 80.264) (end 170.18 90.17) (width 1) (layer B.Cu) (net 7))
 (segment (start 170.18 90.17) (end 120.65 90.17) (width 1) (layer B.Cu) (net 7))
 (segment (start 180.086 71.12) (end 180.086 80.264) (width 1) (layer B.Cu) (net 7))
 (segment (start 213.36 66.04) (end 213.36 59.69) (width 1) (layer B.Cu) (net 8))
 (segment (start 212.09 67.31) (end 213.36 66.04) (width 1) (layer B.Cu) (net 8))
 (segment (start 205.74 67.31) (end 212.09 67.31) (width 1) (layer B.Cu) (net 8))
 (segment (start 204.47 71.12) (end 204.47 68.58) (width 1) (layer B.Cu) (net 8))
 (segment (start 204.47 68.58) (end 205.74 67.31) (width 1) (layer B.Cu) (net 8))
 (segment (start 207.01 71.12) (end 214.63 71.12) (width 1) (layer B.Cu) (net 9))
 (segment (start 215.9 69.85) (end 215.9 59.69) (width 1) (layer B.Cu) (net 9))
 (segment (start 214.63 71.12) (end 215.9 69.85) (width 1) (layer B.Cu) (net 9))
 (segment (start 152.4 118.11) (end 151.13 119.38) (width 1) (layer B.Cu) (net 10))
 (segment (start 156.21 115.57) (end 152.4 118.11) (width 1) (layer B.Cu) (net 10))
 (segment (start 184.15 115.57) (end 156.21 115.57) (width 1) (layer B.Cu) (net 10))
 (via (at 184.15 115.57) (size 2) (layers F.Cu B.Cu) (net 10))
 (segment (start 189.23 115.57) (end 184.15 115.57) (width 1) (layer F.Cu) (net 10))
 (via (at 189.23 115.57) (size 2) (layers F.Cu B.Cu) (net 10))
 (segment (start 193.04 115.57) (end 189.23 115.57) (width 1) (layer B.Cu) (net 10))
 (segment (start 194.31 115.57) (end 193.04 115.57) (width 1) (layer B.Cu) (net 10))
 (segment (start 194.31 119.38) (end 194.31 115.57) (width 1) (layer B.Cu) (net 10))
 (segment (start 151.13 119.38) (end 151.13 129.54) (width 1) (layer B.Cu) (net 10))
 (segment (start 140.97 80.01) (end 168.91 80.01) (width 1) (layer B.Cu) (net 20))
 (segment (start 172.72 76.2) (end 172.72 71.374) (width 1) (layer B.Cu) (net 20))
 (segment (start 168.91 80.01) (end 172.72 76.2) (width 1) (layer B.Cu) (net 20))
 (segment (start 172.72 71.374) (end 172.466 71.12) (width 1) (layer B.Cu) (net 20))
 (segment (start 196.85 71.12) (end 196.85 66.04) (width 1) (layer B.Cu) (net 11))
 (segment (start 189.15 62.15) (end 189.15 59.69) (width 1) (layer B.Cu) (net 11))
 (segment (start 193.04 66.04) (end 189.15 62.15) (width 1) (layer B.Cu) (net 11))
 (segment (start 196.85 66.04) (end 193.04 66.04) (width 1) (layer B.Cu) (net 11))
 (segment (start 201.93 71.12) (end 201.93 66.04) (width 1) (layer B.Cu) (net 12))
 (segment (start 194.15 63.34) (end 194.15 59.69) (width 1) (layer B.Cu) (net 12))
 (segment (start 194.31 63.5) (end 194.15 63.34) (width 1) (layer B.Cu) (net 12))
 (segment (start 199.39 63.5) (end 194.31 63.5) (width 1) (layer B.Cu) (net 12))
 (segment (start 201.93 66.04) (end 199.39 63.5) (width 1) (layer B.Cu) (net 12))
 (segment (start 186.69 68.58) (end 171.45 68.58) (width 1) (layer B.Cu) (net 13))
 (segment (start 171.45 68.58) (end 168.91 66.04) (width 1) (layer B.Cu) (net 13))
 (segment (start 168.91 66.04) (end 158.75 66.04) (width 1) (layer B.Cu) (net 13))
 (segment (start 158.75 66.04) (end 154.94 62.23) (width 1) (layer B.Cu) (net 13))
 (segment (start 154.94 62.23) (end 154.94 59.69) (width 1) (layer B.Cu) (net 13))
 (segment (start 189.23 71.12) (end 186.69 68.58) (width 1) (layer B.Cu) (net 13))
 (segment (start 163.83 63.5) (end 160.02 59.69) (width 1) (layer B.Cu) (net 14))
 (segment (start 170.18 63.5) (end 163.83 63.5) (width 1) (layer B.Cu) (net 14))
 (segment (start 172.72 66.04) (end 170.18 63.5) (width 1) (layer B.Cu) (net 14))
 (segment (start 187.96 66.04) (end 172.72 66.04) (width 1) (layer B.Cu) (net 14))
 (segment (start 191.77 69.85) (end 187.96 66.04) (width 1) (layer B.Cu) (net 14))
 (segment (start 191.77 71.12) (end 191.77 69.85) (width 1) (layer B.Cu) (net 14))
 (segment (start 173.99 129.46) (end 174.07 129.54) (width 1) (layer B.Cu) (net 16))
 (segment (start 196.85 123.19) (end 185.42 123.19) (width 1) (layer B.Cu) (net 16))
 (segment (start 185.42 123.19) (end 182.88 125.73) (width 1) (layer B.Cu) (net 16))
 (segment (start 182.88 125.73) (end 175.26 125.73) (width 1) (layer B.Cu) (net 16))
 (segment (start 175.26 125.73) (end 173.99 127) (width 1) (layer B.Cu) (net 16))
 (segment (start 173.99 127) (end 173.99 129.46) (width 1) (layer B.Cu) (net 16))
 (segment (start 196.85 119.38) (end 196.85 123.19) (width 1) (layer B.Cu) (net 16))
 (segment (start 200.74 128.35) (end 200.74 129.54) (width 1) (layer B.Cu) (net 17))
 (segment (start 199.39 127) (end 200.74 128.35) (width 1) (layer B.Cu) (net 17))
 (segment (start 199.39 119.38) (end 199.39 127) (width 1) (layer B.Cu) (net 17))
 (segment (start 177.546 78.486) (end 170.942 85.09) (width 1) (layer B.Cu) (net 19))
 (segment (start 170.942 85.09) (end 104.14 85.09) (width 1) (layer B.Cu) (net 19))
 (segment (start 104.14 85.09) (end 102.87 83.82) (width 1) (layer B.Cu) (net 19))
 (segment (start 102.87 83.82) (end 102.87 66.04) (width 1) (layer B.Cu) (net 19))
 (segment (start 102.87 66.04) (end 101.6 64.77) (width 1) (layer B.Cu) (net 19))
 (segment (start 101.6 64.77) (end 90.17 64.77) (width 1) (layer B.Cu) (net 19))
 (segment (start 177.546 71.12) (end 177.546 78.486) (width 1) (layer B.Cu) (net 19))
 (segment (start 199.39 81.28) (end 173.99 106.68) (width 1) (layer B.Cu) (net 18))
 (segment (start 173.99 106.68) (end 146.05 106.68) (width 1) (layer B.Cu) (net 18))
 (segment (start 146.05 106.68) (end 132.08 120.65) (width 1) (layer B.Cu) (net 18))
 (segment (start 132.08 120.65) (end 132.08 129.54) (width 1) (layer B.Cu) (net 18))
 (segment (start 199.39 71.12) (end 199.39 81.28) (width 1) (layer B.Cu) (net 18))
 (segment (start 194.31 71.12) (end 194.31 68.58) (width 1) (layer B.Cu) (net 15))
 (segment (start 173.99 63.5) (end 170.18 59.69) (width 1) (layer B.Cu) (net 15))
 (segment (start 187.96 63.5) (end 173.99 63.5) (width 1) (layer B.Cu) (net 15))
 (segment (start 193.04 68.58) (end 187.96 63.5) (width 1) (layer B.Cu) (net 15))
 (segment (start 194.31 68.58) (end 193.04 68.58) (width 1) (layer B.Cu) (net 15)))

